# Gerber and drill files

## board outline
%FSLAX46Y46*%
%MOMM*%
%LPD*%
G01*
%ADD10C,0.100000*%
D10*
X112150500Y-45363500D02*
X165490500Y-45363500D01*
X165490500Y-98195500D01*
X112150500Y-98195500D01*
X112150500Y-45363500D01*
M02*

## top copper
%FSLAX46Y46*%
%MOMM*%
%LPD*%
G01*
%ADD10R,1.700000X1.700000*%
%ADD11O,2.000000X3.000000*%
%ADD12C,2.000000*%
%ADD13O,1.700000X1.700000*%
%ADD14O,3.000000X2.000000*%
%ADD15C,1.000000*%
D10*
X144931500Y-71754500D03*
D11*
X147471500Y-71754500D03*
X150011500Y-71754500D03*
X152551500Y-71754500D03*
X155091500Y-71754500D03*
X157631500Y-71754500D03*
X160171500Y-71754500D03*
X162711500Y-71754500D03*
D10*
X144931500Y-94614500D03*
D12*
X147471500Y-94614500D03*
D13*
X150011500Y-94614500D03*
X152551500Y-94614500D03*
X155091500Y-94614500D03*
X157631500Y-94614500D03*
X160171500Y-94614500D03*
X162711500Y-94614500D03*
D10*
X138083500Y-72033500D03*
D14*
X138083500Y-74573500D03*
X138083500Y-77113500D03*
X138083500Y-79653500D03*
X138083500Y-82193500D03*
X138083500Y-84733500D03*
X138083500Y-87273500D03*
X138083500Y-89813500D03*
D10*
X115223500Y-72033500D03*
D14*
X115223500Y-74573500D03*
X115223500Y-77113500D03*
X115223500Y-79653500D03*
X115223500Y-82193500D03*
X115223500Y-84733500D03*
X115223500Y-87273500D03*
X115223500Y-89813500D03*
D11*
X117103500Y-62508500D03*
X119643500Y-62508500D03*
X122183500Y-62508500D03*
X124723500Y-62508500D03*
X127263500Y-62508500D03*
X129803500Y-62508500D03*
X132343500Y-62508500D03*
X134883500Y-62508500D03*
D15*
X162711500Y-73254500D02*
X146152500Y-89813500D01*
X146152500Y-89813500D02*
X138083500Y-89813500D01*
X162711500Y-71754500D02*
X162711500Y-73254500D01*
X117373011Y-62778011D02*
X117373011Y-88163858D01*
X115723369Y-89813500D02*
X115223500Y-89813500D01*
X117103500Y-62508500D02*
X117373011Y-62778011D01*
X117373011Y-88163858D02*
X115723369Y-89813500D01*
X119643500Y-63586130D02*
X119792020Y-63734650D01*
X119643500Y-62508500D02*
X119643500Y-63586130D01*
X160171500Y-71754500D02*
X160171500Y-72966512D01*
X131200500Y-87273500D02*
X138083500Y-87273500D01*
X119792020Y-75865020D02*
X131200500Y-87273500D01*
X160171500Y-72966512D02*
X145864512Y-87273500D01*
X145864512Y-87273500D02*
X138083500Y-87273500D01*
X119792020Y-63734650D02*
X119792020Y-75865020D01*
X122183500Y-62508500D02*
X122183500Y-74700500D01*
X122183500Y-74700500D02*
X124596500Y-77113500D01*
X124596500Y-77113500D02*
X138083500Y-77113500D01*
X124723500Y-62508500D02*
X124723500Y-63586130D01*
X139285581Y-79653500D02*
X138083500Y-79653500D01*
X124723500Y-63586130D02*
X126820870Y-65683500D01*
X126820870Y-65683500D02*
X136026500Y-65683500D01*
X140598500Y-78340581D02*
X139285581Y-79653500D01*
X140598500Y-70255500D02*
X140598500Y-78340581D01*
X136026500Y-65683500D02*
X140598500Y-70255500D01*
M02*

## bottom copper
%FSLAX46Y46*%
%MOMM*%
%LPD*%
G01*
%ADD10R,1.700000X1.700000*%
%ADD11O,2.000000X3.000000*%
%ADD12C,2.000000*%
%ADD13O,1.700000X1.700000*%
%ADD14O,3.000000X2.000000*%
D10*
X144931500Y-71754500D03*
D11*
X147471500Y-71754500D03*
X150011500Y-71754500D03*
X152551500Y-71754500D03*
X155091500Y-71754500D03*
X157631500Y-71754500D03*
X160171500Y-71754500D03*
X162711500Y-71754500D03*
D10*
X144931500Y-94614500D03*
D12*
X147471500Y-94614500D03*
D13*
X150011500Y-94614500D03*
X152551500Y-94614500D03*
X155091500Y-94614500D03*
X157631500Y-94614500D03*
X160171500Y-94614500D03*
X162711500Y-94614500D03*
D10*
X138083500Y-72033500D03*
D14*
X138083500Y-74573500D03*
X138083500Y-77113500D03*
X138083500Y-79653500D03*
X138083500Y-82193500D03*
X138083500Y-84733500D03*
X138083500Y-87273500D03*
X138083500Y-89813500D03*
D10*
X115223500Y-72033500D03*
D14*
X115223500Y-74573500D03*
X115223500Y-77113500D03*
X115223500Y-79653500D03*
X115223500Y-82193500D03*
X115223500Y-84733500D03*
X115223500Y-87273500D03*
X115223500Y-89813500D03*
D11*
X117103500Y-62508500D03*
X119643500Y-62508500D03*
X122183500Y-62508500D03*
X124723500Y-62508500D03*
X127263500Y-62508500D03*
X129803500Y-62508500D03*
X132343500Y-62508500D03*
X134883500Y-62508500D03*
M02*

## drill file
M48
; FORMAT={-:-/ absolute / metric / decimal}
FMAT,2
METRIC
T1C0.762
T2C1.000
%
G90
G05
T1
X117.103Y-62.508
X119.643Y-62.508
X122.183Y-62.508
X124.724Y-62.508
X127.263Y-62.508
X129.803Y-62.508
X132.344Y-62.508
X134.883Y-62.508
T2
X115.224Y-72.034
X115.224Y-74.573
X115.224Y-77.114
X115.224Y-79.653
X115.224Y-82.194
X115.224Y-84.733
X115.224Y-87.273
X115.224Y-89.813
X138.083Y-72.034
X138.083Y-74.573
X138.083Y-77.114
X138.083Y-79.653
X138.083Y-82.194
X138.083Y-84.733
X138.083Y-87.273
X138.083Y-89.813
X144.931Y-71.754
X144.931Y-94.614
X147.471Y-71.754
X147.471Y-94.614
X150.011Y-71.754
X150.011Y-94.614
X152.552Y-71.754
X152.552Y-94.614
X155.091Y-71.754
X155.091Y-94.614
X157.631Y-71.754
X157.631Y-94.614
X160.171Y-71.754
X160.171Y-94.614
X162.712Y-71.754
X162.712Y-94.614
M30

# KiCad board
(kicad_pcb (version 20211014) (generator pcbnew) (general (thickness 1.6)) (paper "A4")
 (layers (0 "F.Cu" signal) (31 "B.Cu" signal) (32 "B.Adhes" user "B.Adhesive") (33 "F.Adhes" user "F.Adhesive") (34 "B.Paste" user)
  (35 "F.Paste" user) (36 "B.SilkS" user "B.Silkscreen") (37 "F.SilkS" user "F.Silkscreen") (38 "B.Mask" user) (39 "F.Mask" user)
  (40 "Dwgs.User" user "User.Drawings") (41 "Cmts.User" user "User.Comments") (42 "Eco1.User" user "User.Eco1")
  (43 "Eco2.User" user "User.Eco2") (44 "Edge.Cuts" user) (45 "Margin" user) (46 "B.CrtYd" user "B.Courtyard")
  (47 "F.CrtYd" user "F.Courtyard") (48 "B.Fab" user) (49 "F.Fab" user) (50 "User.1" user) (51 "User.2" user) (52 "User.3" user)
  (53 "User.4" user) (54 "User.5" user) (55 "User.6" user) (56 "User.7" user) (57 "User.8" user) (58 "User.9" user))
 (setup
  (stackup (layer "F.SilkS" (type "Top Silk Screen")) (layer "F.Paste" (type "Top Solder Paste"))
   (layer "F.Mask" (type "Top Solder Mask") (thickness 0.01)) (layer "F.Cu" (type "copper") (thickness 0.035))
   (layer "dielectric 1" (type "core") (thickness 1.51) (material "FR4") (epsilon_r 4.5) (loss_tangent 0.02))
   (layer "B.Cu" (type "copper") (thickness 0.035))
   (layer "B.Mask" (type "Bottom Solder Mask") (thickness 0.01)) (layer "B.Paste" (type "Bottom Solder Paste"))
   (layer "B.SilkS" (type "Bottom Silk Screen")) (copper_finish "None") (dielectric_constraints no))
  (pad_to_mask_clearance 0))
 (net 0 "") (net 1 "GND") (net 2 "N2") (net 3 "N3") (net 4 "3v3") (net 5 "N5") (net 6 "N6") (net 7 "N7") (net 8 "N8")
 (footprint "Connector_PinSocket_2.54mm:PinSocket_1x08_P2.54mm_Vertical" (layer "F.Cu") (at 144.9315 71.7545 90)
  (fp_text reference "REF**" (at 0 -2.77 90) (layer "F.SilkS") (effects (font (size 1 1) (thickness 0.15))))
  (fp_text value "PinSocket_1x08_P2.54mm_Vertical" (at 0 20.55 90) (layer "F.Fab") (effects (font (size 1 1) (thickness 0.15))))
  (pad "1" thru_hole rect (at 0 0 90) (size 1.7 1.7) (drill 1) (layers *.Cu *.Mask))
  (pad "2" thru_hole oval (at 0 2.54 90) (size 3 2) (drill 1) (layers *.Cu *.Mask))
  (pad "3" thru_hole oval (at 0 5.08 90) (size 3 2) (drill 1) (layers *.Cu *.Mask))
  (pad "4" thru_hole oval (at 0 7.62 90) (size 3 2) (drill 1) (layers *.Cu *.Mask))
  (pad "5" thru_hole oval (at 0 10.16 90) (size 3 2) (drill 1) (layers *.Cu *.Mask))
  (pad "6" thru_hole oval (at 0 12.7 90) (size 3 2) (drill 1) (layers *.Cu *.Mask))
  (pad "7" thru_hole oval (at 0 15.24 90) (size 3 2) (drill 1) (layers *.Cu *.Mask) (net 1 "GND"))
  (pad "8" thru_hole oval (at 0 17.78 90) (size 3 2) (drill 1) (layers *.Cu *.Mask)))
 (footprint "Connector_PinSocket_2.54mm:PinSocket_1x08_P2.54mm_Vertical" (layer "F.Cu") (at 144.9315 94.6145 90)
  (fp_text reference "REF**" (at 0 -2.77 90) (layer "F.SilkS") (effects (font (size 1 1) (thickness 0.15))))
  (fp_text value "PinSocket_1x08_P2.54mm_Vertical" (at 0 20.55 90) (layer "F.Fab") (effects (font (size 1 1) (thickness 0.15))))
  (pad "1" thru_hole rect (at 0 0 90) (size 1.7 1.7) (drill 1) (layers *.Cu *.Mask))
  (pad "2" thru_hole circle (at 0 2.54 90) (size 2 2) (drill 1) (layers *.Cu *.Mask))
  (pad "3" thru_hole oval (at 0 5.08 90) (size 1.7 1.7) (drill 1) (layers *.Cu *.Mask))
  (pad "4" thru_hole oval (at 0 7.62 90) (size 1.7 1.7) (drill 1) (layers *.Cu *.Mask))
  (pad "5" thru_hole oval (at 0 10.16 90) (size 1.7 1.7) (drill 1) (layers *.Cu *.Mask))
  (pad "6" thru_hole oval (at 0 12.7 90) (size 1.7 1.7) (drill 1) (layers *.Cu *.Mask))
  (pad "7" thru_hole oval (at 0 15.24 90) (size 1.7 1.7) (drill 1) (layers *.Cu *.Mask))
  (pad "8" thru_hole oval (at 0 17.78 90) (size 1.7 1.7) (drill 1) (layers *.Cu *.Mask)))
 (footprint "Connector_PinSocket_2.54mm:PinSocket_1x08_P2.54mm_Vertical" (layer "F.Cu") (at 138.0835 72.0335)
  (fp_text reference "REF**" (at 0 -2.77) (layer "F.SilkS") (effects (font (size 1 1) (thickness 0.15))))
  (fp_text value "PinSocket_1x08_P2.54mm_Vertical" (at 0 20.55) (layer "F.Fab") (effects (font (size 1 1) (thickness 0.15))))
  (pad "1" thru_hole rect (at 0 0) (size 1.7 1.7) (drill 1) (layers *.Cu *.Mask))
  (pad "2" thru_hole oval (at 0 2.54) (size 3 2) (drill 1) (layers *.Cu *.Mask))
  (pad "3" thru_hole oval (at 0 5.08) (size 3 2) (drill 1) (layers *.Cu *.Mask) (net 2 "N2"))
  (pad "4" thru_hole oval (at 0 7.62) (size 3 2) (drill 1) (layers *.Cu *.Mask) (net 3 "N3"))
  (pad "5" thru_hole oval (at 0 10.16) (size 3 2) (drill 1) (layers *.Cu *.Mask))
  (pad "6" thru_hole oval (at 0 12.7) (size 3 2) (drill 1) (layers *.Cu *.Mask))
  (pad "7" thru_hole oval (at 0 15.24) (size 3 2) (drill 1) (layers *.Cu *.Mask) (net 1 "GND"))
  (pad "8" thru_hole oval (at 0 17.78) (size 3 2) (drill 1) (layers *.Cu *.Mask)))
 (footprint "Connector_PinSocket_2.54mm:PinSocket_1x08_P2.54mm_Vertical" (layer "F.Cu") (at 115.2235 72.0335)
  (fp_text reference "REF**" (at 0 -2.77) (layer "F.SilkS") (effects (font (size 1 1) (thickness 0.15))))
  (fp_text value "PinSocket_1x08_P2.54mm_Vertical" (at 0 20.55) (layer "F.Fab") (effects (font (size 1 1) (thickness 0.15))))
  (pad "1" thru_hole rect (at 0 0) (size 1.7 1.7) (drill 1) (layers *.Cu *.Mask))
  (pad "2" thru_hole oval (at 0 2.54) (size 3 2) (drill 1) (layers *.Cu *.Mask))
  (pad "3" thru_hole oval (at 0 5.08) (size 3 2) (drill 1) (layers *.Cu *.Mask))
  (pad "4" thru_hole oval (at 0 7.62) (size 3 2) (drill 1) (layers *.Cu *.Mask))
  (pad "5" thru_hole oval (at 0 10.16) (size 3 2) (drill 1) (layers *.Cu *.Mask))
  (pad "6" thru_hole oval (at 0 12.7) (size 3 2) (drill 1) (layers *.Cu *.Mask))
  (pad "7" thru_hole oval (at 0 15.24) (size 3 2) (drill 1) (layers *.Cu *.Mask))
  (pad "8" thru_hole oval (at 0 17.78) (size 3 2) (drill 1) (layers *.Cu *.Mask) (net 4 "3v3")))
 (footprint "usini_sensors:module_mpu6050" (layer "F.Cu") (at 134.8835 62.5085 90)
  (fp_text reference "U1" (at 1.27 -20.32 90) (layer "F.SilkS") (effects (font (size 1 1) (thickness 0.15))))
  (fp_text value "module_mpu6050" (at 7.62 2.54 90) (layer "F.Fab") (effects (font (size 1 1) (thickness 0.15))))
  (pad "1" thru_hole oval locked (at 0 -17.78 90) (size 3 2) (drill 0.762) (layers *.Cu *.Mask) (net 4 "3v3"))
  (pad "2" thru_hole oval locked (at 0 -15.24 90) (size 3 2) (drill 0.762) (layers *.Cu *.Mask) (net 1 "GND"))
  (pad "3" thru_hole oval locked (at 0 -12.7 90) (size 3 2) (drill 0.762) (layers *.Cu *.Mask) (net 2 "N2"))
  (pad "4" thru_hole oval locked (at 0 -10.16 90) (size 3 2) (drill 0.762) (layers *.Cu *.Mask) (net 3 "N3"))
  (pad "5" thru_hole oval locked (at 0 -7.62 90) (size 3 2) (drill 0.762) (layers *.Cu *.Mask) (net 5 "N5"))
  (pad "6" thru_hole oval locked (at 0 -5.08 90) (size 3 2) (drill 0.762) (layers *.Cu *.Mask) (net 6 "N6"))
  (pad "7" thru_hole oval locked (at 0 -2.54 90) (size 3 2) (drill 0.762) (layers *.Cu *.Mask) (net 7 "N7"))
  (pad "8" thru_hole oval locked (at 0 0 90) (size 3 2) (drill 0.762) (layers *.Cu *.Mask) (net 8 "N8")))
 (gr_rect (start 112.1505 45.3635) (end 165.4905 98.1955) (layer "Edge.Cuts") (width 0.1) (fill none))
 (segment (start 162.7115 73.2545) (end 146.1525 89.8135) (width 1) (layer "F.Cu") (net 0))
 (segment (start 146.1525 89.8135) (end 138.0835 89.8135) (width 1) (layer "F.Cu") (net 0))
 (segment (start 162.7115 71.7545) (end 162.7115 73.2545) (width 1) (layer "F.Cu") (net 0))
 (segment (start 117.373011 62.778011) (end 117.373011 88.163858) (width 1) (layer "F.Cu") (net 4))
 (segment (start 115.723369 89.8135) (end 115.2235 89.8135) (width 1) (layer "F.Cu") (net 4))
 (segment (start 117.1035 62.5085) (end 117.373011 62.778011) (width 1) (layer "F.Cu") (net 4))
 (segment (start 117.373011 88.163858) (end 115.723369 89.8135) (width 1) (layer "F.Cu") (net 4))
 (segment (start 119.6435 63.58613) (end 119.79202 63.73465) (width 1) (layer "F.Cu") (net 1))
 (segment (start 119.6435 62.5085) (end 119.6435 63.58613) (width 1) (layer "F.Cu") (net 1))
 (segment (start 160.1715 71.7545) (end 160.1715 72.966512) (width 1) (layer "F.Cu") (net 1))
 (segment (start 131.2005 87.2735) (end 138.0835 87.2735) (width 1) (layer "F.Cu") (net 1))
 (segment (start 119.79202 75.86502) (end 131.2005 87.2735) (width 1) (layer "F.Cu") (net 1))
 (segment (start 160.1715 72.966512) (end 145.864512 87.2735) (width 1) (layer "F.Cu") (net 1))
 (segment (start 145.864512 87.2735) (end 138.0835 87.2735) (width 1) (layer "F.Cu") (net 1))
 (segment (start 119.79202 63.73465) (end 119.79202 75.86502) (width 1) (layer "F.Cu") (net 1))
 (segment (start 122.1835 62.5085) (end 122.1835 74.7005) (width 1) (layer "F.Cu") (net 2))
 (segment (start 122.1835 74.7005) (end 124.5965 77.1135) (width 1) (layer "F.Cu") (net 2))
 (segment (start 124.5965 77.1135) (end 138.0835 77.1135) (width 1) (layer "F.Cu") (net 2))
 (segment (start 124.7235 62.5085) (end 124.7235 63.58613) (width 1) (layer "F.Cu") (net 3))
 (segment (start 139.285581 79.6535) (end 138.0835 79.6535) (width 1) (layer "F.Cu") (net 3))
 (segment (start 124.7235 63.58613) (end 126.82087 65.6835) (width 1) (layer "F.Cu") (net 3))
 (segment (start 126.82087 65.6835) (end 136.0265 65.6835) (width 1) (layer "F.Cu") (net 3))
 (segment (start 140.5985 78.340581) (end 139.285581 79.6535) (width 1) (layer "F.Cu") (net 3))
 (segment (start 140.5985 70.2555) (end 140.5985 78.340581) (width 1) (layer "F.Cu") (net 3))
 (segment (start 136.0265 65.6835) (end 140.5985 70.2555) (width 1) (layer "F.Cu") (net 3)))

